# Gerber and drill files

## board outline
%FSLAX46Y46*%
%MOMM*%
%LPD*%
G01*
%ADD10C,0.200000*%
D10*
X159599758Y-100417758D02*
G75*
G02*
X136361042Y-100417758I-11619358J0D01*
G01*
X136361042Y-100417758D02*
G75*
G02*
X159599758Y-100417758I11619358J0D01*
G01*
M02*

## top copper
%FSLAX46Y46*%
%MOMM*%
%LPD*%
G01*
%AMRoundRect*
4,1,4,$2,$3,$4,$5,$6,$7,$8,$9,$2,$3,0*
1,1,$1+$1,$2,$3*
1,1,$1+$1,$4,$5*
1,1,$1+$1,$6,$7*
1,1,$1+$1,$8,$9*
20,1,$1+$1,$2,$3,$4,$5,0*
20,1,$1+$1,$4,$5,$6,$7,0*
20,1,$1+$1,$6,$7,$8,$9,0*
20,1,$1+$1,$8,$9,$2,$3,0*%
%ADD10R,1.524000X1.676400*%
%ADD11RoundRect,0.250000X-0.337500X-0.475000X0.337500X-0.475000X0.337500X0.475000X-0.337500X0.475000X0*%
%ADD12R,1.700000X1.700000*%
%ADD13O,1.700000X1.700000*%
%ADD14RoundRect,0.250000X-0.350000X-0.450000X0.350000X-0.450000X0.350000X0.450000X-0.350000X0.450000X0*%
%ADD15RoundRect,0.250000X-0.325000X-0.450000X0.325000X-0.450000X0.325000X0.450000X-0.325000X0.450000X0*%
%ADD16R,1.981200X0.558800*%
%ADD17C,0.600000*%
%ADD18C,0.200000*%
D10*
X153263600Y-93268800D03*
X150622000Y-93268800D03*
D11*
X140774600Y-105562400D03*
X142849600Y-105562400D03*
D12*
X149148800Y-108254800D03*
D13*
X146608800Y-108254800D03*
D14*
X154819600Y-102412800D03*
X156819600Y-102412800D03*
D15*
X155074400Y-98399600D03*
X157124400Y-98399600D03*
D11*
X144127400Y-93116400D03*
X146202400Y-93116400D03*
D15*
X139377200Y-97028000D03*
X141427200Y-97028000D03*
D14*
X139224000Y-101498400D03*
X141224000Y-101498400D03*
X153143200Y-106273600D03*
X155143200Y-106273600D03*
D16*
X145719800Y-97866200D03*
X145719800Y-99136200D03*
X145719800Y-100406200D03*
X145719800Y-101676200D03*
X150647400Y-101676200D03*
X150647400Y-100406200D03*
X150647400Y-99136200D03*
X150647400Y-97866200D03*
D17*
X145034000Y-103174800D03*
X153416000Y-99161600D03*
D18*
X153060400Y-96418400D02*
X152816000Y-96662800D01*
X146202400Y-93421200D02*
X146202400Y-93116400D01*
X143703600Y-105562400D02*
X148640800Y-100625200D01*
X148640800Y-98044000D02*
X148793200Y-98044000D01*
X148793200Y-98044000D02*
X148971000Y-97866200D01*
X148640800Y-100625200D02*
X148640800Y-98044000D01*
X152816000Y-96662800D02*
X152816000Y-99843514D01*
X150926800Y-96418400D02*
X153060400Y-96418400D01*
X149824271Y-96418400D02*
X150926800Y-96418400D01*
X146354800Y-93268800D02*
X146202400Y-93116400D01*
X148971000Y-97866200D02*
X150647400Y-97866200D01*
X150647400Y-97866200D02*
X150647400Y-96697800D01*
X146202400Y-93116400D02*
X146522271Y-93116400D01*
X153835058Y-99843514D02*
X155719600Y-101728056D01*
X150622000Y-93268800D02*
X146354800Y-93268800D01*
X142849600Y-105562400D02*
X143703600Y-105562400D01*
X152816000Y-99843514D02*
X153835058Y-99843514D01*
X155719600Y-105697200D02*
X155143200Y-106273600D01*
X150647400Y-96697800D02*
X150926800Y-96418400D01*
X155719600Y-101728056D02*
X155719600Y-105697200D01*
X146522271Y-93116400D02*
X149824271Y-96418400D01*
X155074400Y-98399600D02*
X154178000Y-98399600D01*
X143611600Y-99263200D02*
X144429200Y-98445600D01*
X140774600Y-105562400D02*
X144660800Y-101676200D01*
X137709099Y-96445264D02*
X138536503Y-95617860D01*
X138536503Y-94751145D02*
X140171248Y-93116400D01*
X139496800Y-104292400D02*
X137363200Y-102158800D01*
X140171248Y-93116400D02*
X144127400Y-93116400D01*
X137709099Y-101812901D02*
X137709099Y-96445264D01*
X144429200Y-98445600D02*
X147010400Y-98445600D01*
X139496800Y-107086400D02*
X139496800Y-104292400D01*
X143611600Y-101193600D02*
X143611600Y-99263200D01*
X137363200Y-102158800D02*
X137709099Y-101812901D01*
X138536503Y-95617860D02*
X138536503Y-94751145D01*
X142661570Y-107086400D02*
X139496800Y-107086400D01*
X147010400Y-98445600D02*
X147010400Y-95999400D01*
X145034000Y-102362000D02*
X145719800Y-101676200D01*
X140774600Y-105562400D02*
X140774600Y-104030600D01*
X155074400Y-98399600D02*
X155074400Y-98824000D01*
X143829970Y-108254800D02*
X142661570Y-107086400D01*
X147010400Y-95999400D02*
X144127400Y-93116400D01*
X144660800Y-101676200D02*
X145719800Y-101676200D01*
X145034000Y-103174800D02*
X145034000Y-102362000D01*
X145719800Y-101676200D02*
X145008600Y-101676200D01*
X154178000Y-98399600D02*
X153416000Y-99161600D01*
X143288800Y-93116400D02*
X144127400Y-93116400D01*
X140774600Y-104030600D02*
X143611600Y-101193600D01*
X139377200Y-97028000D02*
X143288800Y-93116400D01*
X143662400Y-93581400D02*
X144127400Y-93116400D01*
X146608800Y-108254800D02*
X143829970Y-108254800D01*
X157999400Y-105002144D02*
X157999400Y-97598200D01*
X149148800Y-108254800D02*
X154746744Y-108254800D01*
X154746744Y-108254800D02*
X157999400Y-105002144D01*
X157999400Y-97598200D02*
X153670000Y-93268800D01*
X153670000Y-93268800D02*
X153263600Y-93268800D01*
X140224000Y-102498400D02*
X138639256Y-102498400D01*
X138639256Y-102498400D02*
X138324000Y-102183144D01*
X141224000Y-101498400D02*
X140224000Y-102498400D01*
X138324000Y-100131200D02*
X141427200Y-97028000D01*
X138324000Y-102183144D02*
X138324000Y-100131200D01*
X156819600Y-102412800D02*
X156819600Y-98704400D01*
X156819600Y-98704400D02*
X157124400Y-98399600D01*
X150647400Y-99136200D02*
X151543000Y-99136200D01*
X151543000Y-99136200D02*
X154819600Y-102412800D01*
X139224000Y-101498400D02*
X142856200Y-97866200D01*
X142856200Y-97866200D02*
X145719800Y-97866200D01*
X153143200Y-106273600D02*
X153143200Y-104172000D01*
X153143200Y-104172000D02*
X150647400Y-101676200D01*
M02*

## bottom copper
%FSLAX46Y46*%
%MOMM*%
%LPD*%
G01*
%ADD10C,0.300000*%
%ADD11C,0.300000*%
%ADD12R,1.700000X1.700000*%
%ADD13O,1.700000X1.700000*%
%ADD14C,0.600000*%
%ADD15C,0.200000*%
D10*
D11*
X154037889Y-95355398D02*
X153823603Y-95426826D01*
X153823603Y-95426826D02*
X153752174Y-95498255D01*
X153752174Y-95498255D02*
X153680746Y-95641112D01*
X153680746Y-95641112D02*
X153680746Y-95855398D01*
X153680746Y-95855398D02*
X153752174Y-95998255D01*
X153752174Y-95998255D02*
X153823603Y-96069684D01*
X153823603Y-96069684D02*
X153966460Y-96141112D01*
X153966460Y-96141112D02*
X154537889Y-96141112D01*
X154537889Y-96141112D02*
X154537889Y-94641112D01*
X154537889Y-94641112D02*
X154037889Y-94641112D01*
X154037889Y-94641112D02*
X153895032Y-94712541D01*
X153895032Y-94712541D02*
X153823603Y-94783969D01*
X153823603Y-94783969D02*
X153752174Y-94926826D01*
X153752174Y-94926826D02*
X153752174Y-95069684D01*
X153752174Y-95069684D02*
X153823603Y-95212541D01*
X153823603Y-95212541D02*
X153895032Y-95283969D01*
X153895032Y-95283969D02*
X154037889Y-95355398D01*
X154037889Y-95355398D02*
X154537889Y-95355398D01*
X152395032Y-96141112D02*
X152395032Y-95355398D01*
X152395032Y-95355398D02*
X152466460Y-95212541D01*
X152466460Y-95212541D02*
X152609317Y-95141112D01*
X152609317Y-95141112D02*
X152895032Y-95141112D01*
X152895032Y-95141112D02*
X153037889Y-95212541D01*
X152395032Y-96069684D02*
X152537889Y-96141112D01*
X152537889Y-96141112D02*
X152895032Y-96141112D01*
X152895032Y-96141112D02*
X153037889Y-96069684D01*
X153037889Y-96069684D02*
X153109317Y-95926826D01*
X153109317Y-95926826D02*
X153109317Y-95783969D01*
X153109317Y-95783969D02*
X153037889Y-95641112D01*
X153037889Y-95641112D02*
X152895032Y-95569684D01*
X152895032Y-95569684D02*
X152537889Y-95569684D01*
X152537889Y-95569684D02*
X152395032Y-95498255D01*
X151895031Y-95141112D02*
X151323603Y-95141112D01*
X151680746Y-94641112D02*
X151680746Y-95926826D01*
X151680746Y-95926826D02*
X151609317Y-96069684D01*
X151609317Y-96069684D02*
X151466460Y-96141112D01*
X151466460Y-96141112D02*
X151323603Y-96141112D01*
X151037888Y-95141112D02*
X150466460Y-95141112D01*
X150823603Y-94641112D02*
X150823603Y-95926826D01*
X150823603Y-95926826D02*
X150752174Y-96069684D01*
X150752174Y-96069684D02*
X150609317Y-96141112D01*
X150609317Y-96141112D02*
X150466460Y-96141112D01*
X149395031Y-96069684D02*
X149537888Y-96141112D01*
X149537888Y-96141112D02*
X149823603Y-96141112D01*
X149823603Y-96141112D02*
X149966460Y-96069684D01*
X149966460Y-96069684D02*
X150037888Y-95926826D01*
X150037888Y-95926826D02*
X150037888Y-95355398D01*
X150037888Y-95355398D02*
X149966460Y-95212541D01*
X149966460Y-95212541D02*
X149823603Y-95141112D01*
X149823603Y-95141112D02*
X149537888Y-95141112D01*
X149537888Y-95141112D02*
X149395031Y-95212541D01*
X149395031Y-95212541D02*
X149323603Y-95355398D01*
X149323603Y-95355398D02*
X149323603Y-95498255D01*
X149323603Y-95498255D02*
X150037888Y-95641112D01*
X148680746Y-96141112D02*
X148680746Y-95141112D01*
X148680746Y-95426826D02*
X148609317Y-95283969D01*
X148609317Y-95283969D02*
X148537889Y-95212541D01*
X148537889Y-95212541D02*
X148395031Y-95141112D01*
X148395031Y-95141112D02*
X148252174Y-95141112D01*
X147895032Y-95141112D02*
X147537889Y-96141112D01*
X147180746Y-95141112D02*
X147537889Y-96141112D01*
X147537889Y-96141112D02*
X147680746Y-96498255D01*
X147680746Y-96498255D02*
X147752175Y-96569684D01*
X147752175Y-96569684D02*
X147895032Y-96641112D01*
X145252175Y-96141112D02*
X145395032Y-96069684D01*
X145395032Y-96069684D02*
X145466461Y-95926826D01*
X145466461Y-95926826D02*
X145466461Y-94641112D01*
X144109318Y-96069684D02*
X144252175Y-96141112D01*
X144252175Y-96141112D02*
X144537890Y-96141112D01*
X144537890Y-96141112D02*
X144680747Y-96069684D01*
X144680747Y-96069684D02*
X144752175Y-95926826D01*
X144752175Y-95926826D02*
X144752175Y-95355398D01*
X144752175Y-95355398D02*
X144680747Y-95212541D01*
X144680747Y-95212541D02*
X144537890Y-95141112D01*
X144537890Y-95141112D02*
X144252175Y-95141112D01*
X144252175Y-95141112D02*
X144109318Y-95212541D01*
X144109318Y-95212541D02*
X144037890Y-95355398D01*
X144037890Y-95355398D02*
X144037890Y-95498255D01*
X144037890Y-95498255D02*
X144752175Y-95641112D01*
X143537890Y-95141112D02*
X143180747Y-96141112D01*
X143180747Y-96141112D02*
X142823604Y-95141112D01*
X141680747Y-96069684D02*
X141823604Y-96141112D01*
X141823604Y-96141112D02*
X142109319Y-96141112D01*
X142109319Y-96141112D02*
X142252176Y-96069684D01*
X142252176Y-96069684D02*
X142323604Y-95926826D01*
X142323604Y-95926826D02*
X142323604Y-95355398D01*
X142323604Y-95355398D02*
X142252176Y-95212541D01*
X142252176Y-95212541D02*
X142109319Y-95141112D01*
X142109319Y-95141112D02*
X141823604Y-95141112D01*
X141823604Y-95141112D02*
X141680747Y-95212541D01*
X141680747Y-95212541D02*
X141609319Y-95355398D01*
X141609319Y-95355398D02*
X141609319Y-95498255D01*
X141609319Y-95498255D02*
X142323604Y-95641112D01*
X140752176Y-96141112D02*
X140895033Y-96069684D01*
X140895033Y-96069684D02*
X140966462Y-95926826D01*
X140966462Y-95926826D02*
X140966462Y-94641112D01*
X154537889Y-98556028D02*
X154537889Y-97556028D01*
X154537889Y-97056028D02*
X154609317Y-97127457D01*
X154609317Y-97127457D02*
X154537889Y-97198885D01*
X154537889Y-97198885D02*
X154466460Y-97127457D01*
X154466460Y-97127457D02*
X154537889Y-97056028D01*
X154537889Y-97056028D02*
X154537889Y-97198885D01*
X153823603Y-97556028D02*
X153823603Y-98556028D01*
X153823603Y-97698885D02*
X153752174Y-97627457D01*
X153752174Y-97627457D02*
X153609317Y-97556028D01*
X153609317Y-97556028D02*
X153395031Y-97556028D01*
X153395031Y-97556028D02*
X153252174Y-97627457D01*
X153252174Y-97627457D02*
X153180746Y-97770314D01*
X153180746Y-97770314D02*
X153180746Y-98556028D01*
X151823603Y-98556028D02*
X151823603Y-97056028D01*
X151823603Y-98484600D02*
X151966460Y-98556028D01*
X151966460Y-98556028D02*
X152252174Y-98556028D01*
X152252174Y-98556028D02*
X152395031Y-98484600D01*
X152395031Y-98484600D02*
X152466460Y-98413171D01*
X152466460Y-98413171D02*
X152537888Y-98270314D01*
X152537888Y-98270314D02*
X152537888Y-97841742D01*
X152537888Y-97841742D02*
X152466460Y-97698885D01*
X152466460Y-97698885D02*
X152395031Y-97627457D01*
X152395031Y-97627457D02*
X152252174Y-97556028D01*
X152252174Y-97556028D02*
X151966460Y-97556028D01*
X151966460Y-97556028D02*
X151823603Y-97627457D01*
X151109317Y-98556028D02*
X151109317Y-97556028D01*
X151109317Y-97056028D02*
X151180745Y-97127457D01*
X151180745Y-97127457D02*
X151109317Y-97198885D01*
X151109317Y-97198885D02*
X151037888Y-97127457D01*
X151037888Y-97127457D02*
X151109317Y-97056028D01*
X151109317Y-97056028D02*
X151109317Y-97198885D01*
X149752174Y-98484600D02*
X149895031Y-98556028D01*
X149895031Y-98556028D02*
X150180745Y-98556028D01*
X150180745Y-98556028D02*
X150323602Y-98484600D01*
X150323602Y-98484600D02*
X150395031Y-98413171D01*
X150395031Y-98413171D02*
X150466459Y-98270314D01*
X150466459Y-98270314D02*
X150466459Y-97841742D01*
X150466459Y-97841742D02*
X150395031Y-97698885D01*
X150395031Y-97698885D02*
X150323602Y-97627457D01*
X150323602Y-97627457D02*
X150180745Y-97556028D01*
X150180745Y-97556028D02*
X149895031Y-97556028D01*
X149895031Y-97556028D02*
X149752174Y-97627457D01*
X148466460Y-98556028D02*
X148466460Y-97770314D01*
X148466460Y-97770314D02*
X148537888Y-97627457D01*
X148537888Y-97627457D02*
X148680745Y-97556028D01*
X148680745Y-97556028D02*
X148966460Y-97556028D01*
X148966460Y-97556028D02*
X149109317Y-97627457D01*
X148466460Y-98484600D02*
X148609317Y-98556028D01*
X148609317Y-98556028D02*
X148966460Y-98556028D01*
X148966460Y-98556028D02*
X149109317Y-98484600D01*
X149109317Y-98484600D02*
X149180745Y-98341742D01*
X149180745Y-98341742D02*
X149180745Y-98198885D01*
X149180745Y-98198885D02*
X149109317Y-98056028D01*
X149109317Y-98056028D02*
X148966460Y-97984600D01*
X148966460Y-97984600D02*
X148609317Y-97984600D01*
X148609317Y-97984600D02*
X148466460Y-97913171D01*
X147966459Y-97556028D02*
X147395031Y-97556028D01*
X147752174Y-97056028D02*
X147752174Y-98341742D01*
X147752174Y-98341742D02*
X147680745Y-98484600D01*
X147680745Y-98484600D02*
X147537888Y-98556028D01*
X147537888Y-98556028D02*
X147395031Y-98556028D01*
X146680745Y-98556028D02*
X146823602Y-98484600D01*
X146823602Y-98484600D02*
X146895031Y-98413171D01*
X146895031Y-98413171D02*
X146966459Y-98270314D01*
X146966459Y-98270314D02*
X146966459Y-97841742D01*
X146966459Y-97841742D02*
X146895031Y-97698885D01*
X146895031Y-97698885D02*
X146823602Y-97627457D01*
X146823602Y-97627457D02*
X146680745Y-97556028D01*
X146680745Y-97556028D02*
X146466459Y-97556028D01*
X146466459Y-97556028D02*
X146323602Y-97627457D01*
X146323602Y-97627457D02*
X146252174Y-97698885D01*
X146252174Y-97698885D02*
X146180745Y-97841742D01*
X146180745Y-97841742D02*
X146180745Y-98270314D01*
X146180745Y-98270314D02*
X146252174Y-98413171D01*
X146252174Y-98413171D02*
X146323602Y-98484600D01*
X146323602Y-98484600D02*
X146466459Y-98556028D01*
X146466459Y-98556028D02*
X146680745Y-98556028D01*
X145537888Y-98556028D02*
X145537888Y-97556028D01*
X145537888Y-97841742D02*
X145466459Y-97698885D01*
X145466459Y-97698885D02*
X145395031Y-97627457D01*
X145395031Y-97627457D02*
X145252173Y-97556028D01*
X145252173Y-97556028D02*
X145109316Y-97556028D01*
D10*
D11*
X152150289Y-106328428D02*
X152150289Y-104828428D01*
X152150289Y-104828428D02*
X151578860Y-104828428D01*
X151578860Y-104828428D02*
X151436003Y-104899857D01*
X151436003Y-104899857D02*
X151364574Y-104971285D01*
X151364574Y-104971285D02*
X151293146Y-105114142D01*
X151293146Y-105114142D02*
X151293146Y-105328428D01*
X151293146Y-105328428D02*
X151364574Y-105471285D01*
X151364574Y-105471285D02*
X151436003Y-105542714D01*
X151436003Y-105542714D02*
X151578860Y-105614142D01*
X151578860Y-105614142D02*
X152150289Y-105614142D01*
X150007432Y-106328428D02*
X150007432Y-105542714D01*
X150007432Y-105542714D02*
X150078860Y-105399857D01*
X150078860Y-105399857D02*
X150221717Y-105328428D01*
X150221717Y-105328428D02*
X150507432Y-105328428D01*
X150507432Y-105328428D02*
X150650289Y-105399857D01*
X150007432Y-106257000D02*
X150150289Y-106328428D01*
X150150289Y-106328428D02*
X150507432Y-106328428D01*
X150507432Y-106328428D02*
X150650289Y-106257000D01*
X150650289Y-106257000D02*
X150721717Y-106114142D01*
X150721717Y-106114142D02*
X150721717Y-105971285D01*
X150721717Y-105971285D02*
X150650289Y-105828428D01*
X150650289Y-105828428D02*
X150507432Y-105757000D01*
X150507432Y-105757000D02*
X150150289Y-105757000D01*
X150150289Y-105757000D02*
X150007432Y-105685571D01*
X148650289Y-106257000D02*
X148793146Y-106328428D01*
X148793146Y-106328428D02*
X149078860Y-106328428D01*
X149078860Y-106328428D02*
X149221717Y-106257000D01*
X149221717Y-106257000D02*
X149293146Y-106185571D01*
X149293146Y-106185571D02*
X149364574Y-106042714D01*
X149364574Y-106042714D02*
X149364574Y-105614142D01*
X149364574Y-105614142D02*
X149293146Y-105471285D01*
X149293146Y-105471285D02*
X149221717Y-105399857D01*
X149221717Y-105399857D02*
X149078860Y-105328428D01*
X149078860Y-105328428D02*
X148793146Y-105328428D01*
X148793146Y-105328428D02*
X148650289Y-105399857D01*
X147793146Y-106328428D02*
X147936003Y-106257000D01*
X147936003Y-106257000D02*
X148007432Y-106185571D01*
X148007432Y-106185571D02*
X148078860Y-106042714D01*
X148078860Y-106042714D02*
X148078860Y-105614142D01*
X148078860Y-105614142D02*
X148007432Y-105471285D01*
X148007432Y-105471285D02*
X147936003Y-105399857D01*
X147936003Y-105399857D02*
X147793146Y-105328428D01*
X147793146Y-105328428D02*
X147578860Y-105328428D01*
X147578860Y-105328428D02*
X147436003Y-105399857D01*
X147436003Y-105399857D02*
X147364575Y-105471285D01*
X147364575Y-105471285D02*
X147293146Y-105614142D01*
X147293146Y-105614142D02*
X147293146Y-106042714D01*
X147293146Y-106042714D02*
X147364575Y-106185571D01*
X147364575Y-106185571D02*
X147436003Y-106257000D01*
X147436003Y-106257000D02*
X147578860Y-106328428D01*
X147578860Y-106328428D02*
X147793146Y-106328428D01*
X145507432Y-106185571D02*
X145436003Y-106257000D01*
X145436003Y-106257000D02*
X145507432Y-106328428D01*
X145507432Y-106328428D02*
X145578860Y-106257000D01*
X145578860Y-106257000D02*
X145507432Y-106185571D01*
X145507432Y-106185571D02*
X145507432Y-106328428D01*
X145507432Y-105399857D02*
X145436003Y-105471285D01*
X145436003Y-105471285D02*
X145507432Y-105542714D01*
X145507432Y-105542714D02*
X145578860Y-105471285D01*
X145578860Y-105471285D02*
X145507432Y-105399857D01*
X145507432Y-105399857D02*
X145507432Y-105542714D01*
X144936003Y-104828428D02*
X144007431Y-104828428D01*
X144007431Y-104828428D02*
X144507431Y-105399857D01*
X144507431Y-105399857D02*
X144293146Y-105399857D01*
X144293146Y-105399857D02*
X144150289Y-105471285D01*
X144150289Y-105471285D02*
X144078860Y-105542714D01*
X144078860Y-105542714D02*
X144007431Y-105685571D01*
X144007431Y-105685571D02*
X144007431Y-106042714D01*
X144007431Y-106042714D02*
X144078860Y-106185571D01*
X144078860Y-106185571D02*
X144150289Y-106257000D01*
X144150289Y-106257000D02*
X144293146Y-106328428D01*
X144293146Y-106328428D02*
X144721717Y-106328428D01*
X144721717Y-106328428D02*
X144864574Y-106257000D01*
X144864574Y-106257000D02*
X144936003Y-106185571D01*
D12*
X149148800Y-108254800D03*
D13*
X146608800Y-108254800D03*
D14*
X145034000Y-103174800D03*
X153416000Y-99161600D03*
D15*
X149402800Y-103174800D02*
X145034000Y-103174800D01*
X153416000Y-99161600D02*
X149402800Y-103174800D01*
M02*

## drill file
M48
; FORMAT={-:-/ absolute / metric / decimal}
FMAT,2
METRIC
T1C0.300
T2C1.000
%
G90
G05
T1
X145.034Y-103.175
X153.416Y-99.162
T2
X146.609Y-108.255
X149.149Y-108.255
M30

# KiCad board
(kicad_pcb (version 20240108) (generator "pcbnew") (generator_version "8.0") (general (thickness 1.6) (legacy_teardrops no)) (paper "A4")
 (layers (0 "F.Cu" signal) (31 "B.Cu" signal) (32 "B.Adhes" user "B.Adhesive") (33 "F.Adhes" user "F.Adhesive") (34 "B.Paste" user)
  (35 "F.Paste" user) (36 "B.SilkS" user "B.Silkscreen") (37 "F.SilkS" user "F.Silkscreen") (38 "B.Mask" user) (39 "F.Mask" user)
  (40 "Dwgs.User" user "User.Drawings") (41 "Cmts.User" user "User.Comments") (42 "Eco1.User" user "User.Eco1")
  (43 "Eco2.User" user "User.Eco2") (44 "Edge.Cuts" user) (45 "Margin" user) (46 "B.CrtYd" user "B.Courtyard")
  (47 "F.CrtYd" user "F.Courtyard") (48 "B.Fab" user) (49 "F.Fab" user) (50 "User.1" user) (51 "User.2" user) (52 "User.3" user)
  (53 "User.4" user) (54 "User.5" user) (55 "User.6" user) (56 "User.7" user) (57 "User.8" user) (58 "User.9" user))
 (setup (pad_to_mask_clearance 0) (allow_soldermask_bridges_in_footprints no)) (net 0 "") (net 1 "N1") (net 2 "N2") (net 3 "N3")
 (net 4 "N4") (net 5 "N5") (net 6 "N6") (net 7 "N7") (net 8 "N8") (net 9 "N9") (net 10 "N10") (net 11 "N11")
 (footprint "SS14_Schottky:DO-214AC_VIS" (layer "F.Cu") (at 151.9428 93.2688 180)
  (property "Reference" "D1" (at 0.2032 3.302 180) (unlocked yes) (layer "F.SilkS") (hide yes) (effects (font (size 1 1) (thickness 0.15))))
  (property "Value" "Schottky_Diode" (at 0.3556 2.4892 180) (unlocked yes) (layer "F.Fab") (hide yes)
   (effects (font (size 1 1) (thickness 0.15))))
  (pad "1" smd rect (at -1.3208 0 180) (size 1.524 1.6764) (layers "F.Cu" "F.Paste" "F.Mask") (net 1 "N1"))
  (pad "2" smd rect (at 1.3208 0 180) (size 1.524 1.6764) (layers "F.Cu" "F.Paste" "F.Mask") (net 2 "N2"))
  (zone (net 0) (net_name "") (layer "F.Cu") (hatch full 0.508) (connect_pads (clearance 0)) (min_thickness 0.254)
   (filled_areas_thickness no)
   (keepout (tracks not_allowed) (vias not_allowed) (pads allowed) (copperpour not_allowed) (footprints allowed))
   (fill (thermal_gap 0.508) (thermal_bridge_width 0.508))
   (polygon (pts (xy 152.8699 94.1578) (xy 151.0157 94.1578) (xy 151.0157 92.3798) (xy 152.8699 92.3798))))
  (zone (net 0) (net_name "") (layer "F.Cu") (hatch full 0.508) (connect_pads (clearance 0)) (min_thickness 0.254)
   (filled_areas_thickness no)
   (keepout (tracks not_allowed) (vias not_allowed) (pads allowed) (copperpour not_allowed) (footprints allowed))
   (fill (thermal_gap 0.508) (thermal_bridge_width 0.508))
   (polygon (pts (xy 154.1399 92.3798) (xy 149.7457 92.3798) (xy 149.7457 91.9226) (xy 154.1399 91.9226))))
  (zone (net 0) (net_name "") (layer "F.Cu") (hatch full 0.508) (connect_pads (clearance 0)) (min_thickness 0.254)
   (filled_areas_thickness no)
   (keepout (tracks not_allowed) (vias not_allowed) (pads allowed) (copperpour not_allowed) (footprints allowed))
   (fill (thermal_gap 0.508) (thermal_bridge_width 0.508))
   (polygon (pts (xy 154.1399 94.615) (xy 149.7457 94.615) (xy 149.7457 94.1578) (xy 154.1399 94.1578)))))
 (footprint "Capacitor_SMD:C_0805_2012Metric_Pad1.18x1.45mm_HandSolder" (layer "F.Cu") (at 141.8121 105.5624)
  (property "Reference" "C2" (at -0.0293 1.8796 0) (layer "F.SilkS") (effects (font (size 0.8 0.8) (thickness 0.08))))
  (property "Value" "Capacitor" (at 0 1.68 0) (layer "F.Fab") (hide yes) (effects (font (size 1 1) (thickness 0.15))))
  (pad "1" smd roundrect (at -1.0375 0) (size 1.175 1.45) (layers "F.Cu" "F.Paste" "F.Mask") (roundrect_rratio 0.212766) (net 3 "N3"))
  (pad "2" smd roundrect (at 1.0375 0) (size 1.175 1.45) (layers "F.Cu" "F.Paste" "F.Mask") (roundrect_rratio 0.212766) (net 2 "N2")))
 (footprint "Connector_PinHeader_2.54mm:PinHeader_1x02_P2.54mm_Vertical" (layer "F.Cu") (at 149.1488 108.2548 -90)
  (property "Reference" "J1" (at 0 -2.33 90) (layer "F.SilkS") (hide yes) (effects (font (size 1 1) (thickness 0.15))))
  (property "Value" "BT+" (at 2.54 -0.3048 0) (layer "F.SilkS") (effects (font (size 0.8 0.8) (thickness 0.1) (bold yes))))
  (pad "1" thru_hole rect (at 0 0 270) (size 1.7 1.7) (drill 1) (layers "*.Cu" "*.Mask") (remove_unused_layers no) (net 1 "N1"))
  (pad "2" thru_hole oval (at 0 2.54 270) (size 1.7 1.7) (drill 1) (layers "*.Cu" "*.Mask") (remove_unused_layers no) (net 3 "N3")))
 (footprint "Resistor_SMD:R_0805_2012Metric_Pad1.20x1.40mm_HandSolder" (layer "F.Cu") (at 155.8196 102.4128)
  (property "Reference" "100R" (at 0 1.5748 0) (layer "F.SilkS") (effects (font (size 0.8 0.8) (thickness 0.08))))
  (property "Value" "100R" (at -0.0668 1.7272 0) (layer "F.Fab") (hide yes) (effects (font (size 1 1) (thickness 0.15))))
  (pad "1" smd roundrect (at -1 0) (size 1.2 1.4) (layers "F.Cu" "F.Paste" "F.Mask") (roundrect_rratio 0.208333) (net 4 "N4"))
  (pad "2" smd roundrect (at 1 0) (size 1.2 1.4) (layers "F.Cu" "F.Paste" "F.Mask") (roundrect_rratio 0.208333) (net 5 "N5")))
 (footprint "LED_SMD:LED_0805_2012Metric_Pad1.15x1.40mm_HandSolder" (layer "F.Cu") (at 156.0994 98.3996)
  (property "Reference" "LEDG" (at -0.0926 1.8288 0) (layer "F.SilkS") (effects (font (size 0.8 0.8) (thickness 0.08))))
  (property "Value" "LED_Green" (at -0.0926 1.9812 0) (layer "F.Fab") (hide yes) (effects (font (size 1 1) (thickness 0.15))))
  (pad "1" smd roundrect (at -1.025 0) (size 1.15 1.4) (layers "F.Cu" "F.Paste" "F.Mask") (roundrect_rratio 0.217391) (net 3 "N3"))
  (pad "2" smd roundrect (at 1.025 0) (size 1.15 1.4) (layers "F.Cu" "F.Paste" "F.Mask") (roundrect_rratio 0.217391) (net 5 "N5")))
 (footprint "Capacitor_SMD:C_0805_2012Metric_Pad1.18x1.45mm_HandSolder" (layer "F.Cu") (at 145.1649 93.1164)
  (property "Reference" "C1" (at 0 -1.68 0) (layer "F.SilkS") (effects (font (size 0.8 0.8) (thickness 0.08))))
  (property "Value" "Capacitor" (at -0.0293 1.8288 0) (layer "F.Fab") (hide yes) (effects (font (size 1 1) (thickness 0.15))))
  (pad "1" smd roundrect (at -1.0375 0) (size 1.175 1.45) (layers "F.Cu" "F.Paste" "F.Mask") (roundrect_rratio 0.212766) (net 3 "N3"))
  (pad "2" smd roundrect (at 1.0375 0) (size 1.175 1.45) (layers "F.Cu" "F.Paste" "F.Mask") (roundrect_rratio 0.212766) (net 2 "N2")))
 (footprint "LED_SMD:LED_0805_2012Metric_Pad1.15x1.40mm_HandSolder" (layer "F.Cu") (at 140.4022 97.028)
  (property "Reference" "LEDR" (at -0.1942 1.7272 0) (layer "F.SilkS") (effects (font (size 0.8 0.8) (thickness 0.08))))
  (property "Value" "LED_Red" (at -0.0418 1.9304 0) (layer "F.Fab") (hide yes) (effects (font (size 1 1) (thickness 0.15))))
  (pad "1" smd roundrect (at -1.025 0) (size 1.15 1.4) (layers "F.Cu" "F.Paste" "F.Mask") (roundrect_rratio 0.217391) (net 3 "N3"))
  (pad "2" smd roundrect (at 1.025 0) (size 1.15 1.4) (layers "F.Cu" "F.Paste" "F.Mask") (roundrect_rratio 0.217391) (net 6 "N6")))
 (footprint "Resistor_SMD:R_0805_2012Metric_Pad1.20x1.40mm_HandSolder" (layer "F.Cu") (at 140.224 101.4984)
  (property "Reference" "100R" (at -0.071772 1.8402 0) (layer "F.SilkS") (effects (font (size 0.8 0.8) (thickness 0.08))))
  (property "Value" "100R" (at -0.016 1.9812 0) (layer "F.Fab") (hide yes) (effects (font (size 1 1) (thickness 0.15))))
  (pad "1" smd roundrect (at -1 0) (size 1.2 1.4) (layers "F.Cu" "F.Paste" "F.Mask") (roundrect_rratio 0.208333) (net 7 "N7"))
  (pad "2" smd roundrect (at 1 0) (size 1.2 1.4) (layers "F.Cu" "F.Paste" "F.Mask") (roundrect_rratio 0.208333) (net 6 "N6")))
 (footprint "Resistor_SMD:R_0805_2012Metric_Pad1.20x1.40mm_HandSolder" (layer "F.Cu") (at 154.1432 106.2736)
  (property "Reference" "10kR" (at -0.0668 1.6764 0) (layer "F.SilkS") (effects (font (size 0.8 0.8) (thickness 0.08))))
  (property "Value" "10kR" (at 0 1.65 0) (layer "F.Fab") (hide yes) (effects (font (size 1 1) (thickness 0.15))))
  (pad "1" smd roundrect (at -1 0) (size 1.2 1.4) (layers "F.Cu" "F.Paste" "F.Mask") (roundrect_rratio 0.208333) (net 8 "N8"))
  (pad "2" smd roundrect (at 1 0) (size 1.2 1.4) (layers "F.Cu" "F.Paste" "F.Mask") (roundrect_rratio 0.208333) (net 2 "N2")))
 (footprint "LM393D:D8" (layer "F.Cu") (at 148.1836 99.7712)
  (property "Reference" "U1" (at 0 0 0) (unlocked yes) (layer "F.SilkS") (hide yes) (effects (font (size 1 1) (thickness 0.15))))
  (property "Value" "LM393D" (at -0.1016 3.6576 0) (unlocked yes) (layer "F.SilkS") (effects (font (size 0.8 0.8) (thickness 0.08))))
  (pad "1" smd rect (at -2.4638 -1.905) (size 1.9812 0.5588) (layers "F.Cu" "F.Paste" "F.Mask") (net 7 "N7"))
  (pad "2" smd rect (at -2.4638 -0.635) (size 1.9812 0.5588) (layers "F.Cu" "F.Paste" "F.Mask") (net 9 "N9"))
  (pad "3" smd rect (at -2.4638 0.635) (size 1.9812 0.5588) (layers "F.Cu" "F.Paste" "F.Mask") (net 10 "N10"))
  (pad "4" smd rect (at -2.4638 1.905) (size 1.9812 0.5588) (layers "F.Cu" "F.Paste" "F.Mask") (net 3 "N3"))
  (pad "5" smd rect (at 2.4638 1.905) (size 1.9812 0.5588) (layers "F.Cu" "F.Paste" "F.Mask") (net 8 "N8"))
  (pad "6" smd rect (at 2.4638 0.635) (size 1.9812 0.5588) (layers "F.Cu" "F.Paste" "F.Mask") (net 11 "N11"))
  (pad "7" smd rect (at 2.4638 -0.635) (size 1.9812 0.5588) (layers "F.Cu" "F.Paste" "F.Mask") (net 4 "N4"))
  (pad "8" smd rect (at 2.4638 -1.905) (size 1.9812 0.5588) (layers "F.Cu" "F.Paste" "F.Mask") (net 2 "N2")))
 (gr_circle (center 147.9804 100.417758) (end 159.599758 100.417758) (stroke (width 0.2) (type default)) (fill none) (layer "Edge.Cuts"))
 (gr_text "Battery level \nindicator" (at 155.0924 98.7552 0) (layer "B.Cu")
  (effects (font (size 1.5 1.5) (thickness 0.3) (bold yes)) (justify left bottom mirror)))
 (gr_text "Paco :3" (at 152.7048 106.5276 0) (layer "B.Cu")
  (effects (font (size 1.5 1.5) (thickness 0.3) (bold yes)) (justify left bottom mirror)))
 (segment (start 153.0604 96.4184) (end 152.816 96.6628) (width 0.2) (layer "F.Cu") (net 2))
 (segment (start 146.2024 93.4212) (end 146.2024 93.1164) (width 0.2) (layer "F.Cu") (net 2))
 (segment (start 143.7036 105.5624) (end 148.6408 100.6252) (width 0.2) (layer "F.Cu") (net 2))
 (segment (start 148.6408 98.044) (end 148.7932 98.044) (width 0.2) (layer "F.Cu") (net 2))
 (segment (start 148.7932 98.044) (end 148.971 97.8662) (width 0.2) (layer "F.Cu") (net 2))
 (segment (start 148.6408 100.6252) (end 148.6408 98.044) (width 0.2) (layer "F.Cu") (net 2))
 (segment (start 152.816 96.6628) (end 152.816 99.843514) (width 0.2) (layer "F.Cu") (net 2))
 (segment (start 150.9268 96.4184) (end 153.0604 96.4184) (width 0.2) (layer "F.Cu") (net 2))
 (segment (start 149.824271 96.4184) (end 150.9268 96.4184) (width 0.2) (layer "F.Cu") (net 2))
 (segment (start 146.3548 93.2688) (end 146.2024 93.1164) (width 0.2) (layer "F.Cu") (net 2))
 (segment (start 148.971 97.8662) (end 150.6474 97.8662) (width 0.2) (layer "F.Cu") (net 2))
 (segment (start 150.6474 97.8662) (end 150.6474 96.6978) (width 0.2) (layer "F.Cu") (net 2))
 (segment (start 146.2024 93.1164) (end 146.522271 93.1164) (width 0.2) (layer "F.Cu") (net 2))
 (segment (start 153.835058 99.843514) (end 155.7196 101.728056) (width 0.2) (layer "F.Cu") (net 2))
 (segment (start 150.622 93.2688) (end 146.3548 93.2688) (width 0.2) (layer "F.Cu") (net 2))
 (segment (start 142.8496 105.5624) (end 143.7036 105.5624) (width 0.2) (layer "F.Cu") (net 2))
 (segment (start 152.816 99.843514) (end 153.835058 99.843514) (width 0.2) (layer "F.Cu") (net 2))
 (segment (start 155.7196 105.6972) (end 155.1432 106.2736) (width 0.2) (layer "F.Cu") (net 2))
 (segment (start 150.6474 96.6978) (end 150.9268 96.4184) (width 0.2) (layer "F.Cu") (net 2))
 (segment (start 155.7196 101.728056) (end 155.7196 105.6972) (width 0.2) (layer "F.Cu") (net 2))
 (segment (start 146.522271 93.1164) (end 149.824271 96.4184) (width 0.2) (layer "F.Cu") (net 2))
 (segment (start 155.0744 98.3996) (end 154.178 98.3996) (width 0.2) (layer "F.Cu") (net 3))
 (segment (start 143.6116 99.2632) (end 144.4292 98.4456) (width 0.2) (layer "F.Cu") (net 3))
 (segment (start 140.7746 105.5624) (end 144.6608 101.6762) (width 0.2) (layer "F.Cu") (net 3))
 (segment (start 137.709099 96.445264) (end 138.536503 95.61786) (width 0.2) (layer "F.Cu") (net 3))
 (segment (start 138.536503 94.751145) (end 140.171248 93.1164) (width 0.2) (layer "F.Cu") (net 3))
 (segment (start 139.4968 104.2924) (end 137.3632 102.1588) (width 0.2) (layer "F.Cu") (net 3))
 (segment (start 140.171248 93.1164) (end 144.1274 93.1164) (width 0.2) (layer "F.Cu") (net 3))
 (segment (start 137.709099 101.812901) (end 137.709099 96.445264) (width 0.2) (layer "F.Cu") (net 3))
 (segment (start 144.4292 98.4456) (end 147.0104 98.4456) (width 0.2) (layer "F.Cu") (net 3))
 (segment (start 139.4968 107.0864) (end 139.4968 104.2924) (width 0.2) (layer "F.Cu") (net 3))
 (segment (start 143.6116 101.1936) (end 143.6116 99.2632) (width 0.2) (layer "F.Cu") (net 3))
 (segment (start 137.3632 102.1588) (end 137.709099 101.812901) (width 0.2) (layer "F.Cu") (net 3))
 (segment (start 138.536503 95.61786) (end 138.536503 94.751145) (width 0.2) (layer "F.Cu") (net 3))
 (segment (start 142.66157 107.0864) (end 139.4968 107.0864) (width 0.2) (layer "F.Cu") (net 3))
 (segment (start 147.0104 98.4456) (end 147.0104 95.9994) (width 0.2) (layer "F.Cu") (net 3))
 (segment (start 145.034 102.362) (end 145.7198 101.6762) (width 0.2) (layer "F.Cu") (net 3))
 (segment (start 140.7746 105.5624) (end 140.7746 104.0306) (width 0.2) (layer "F.Cu") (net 3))
 (segment (start 155.0744 98.3996) (end 155.0744 98.824) (width 0.2) (layer "F.Cu") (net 3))
 (segment (start 143.82997 108.2548) (end 142.66157 107.0864) (width 0.2) (layer "F.Cu") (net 3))
 (segment (start 147.0104 95.9994) (end 144.1274 93.1164) (width 0.2) (layer "F.Cu") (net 3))
 (segment (start 144.6608 101.6762) (end 145.7198 101.6762) (width 0.2) (layer "F.Cu") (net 3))
 (segment (start 145.034 103.1748) (end 145.034 102.362) (width 0.2) (layer "F.Cu") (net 3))
 (segment (start 145.7198 101.6762) (end 145.0086 101.6762) (width 0.2) (layer "F.Cu") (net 3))
 (segment (start 154.178 98.3996) (end 153.416 99.1616) (width 0.2) (layer "F.Cu") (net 3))
 (segment (start 143.2888 93.1164) (end 144.1274 93.1164) (width 0.2) (layer "F.Cu") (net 3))
 (segment (start 140.7746 104.0306) (end 143.6116 101.1936) (width 0.2) (layer "F.Cu") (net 3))
 (segment (start 139.3772 97.028) (end 143.2888 93.1164) (width 0.2) (layer "F.Cu") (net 3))
 (segment (start 143.6624 93.5814) (end 144.1274 93.1164) (width 0.2) (layer "F.Cu") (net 3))
 (segment (start 146.6088 108.2548) (end 143.82997 108.2548) (width 0.2) (layer "F.Cu") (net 3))
 (via (at 145.034 103.1748) (size 0.6) (drill 0.3) (layers "F.Cu" "B.Cu") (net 3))
 (via (at 153.416 99.1616) (size 0.6) (drill 0.3) (layers "F.Cu" "B.Cu") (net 3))
 (segment (start 149.4028 103.1748) (end 145.034 103.1748) (width 0.2) (layer "B.Cu") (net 3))
 (segment (start 153.416 99.1616) (end 149.4028 103.1748) (width 0.2) (layer "B.Cu") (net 3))
 (segment (start 157.9994 105.002144) (end 157.9994 97.5982) (width 0.2) (layer "F.Cu") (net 1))
 (segment (start 149.1488 108.2548) (end 154.746744 108.2548) (width 0.2) (layer "F.Cu") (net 1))
 (segment (start 154.746744 108.2548) (end 157.9994 105.002144) (width 0.2) (layer "F.Cu") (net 1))
 (segment (start 157.9994 97.5982) (end 153.67 93.2688) (width 0.2) (layer "F.Cu") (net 1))
 (segment (start 153.67 93.2688) (end 153.2636 93.2688) (width 0.2) (layer "F.Cu") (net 1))
 (segment (start 140.224 102.4984) (end 138.639256 102.4984) (width 0.2) (layer "F.Cu") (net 6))
 (segment (start 138.639256 102.4984) (end 138.324 102.183144) (width 0.2) (layer "F.Cu") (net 6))
 (segment (start 141.224 101.4984) (end 140.224 102.4984) (width 0.2) (layer "F.Cu") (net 6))
 (segment (start 138.324 100.1312) (end 141.4272 97.028) (width 0.2) (layer "F.Cu") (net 6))
 (segment (start 138.324 102.183144) (end 138.324 100.1312) (width 0.2) (layer "F.Cu") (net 6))
 (segment (start 156.8196 102.4128) (end 156.8196 98.7044) (width 0.2) (layer "F.Cu") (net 5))
 (segment (start 156.8196 98.7044) (end 157.1244 98.3996) (width 0.2) (layer "F.Cu") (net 5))
 (segment (start 150.6474 99.1362) (end 151.543 99.1362) (width 0.2) (layer "F.Cu") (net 4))
 (segment (start 151.543 99.1362) (end 154.8196 102.4128) (width 0.2) (layer "F.Cu") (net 4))
 (segment (start 139.224 101.4984) (end 142.8562 97.8662) (width 0.2) (layer "F.Cu") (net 7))
 (segment (start 142.8562 97.8662) (end 145.7198 97.8662) (width 0.2) (layer "F.Cu") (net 7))
 (segment (start 153.1432 106.2736) (end 153.1432 104.172) (width 0.2) (layer "F.Cu") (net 8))
 (segment (start 153.1432 104.172) (end 150.6474 101.6762) (width 0.2) (layer "F.Cu") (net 8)))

